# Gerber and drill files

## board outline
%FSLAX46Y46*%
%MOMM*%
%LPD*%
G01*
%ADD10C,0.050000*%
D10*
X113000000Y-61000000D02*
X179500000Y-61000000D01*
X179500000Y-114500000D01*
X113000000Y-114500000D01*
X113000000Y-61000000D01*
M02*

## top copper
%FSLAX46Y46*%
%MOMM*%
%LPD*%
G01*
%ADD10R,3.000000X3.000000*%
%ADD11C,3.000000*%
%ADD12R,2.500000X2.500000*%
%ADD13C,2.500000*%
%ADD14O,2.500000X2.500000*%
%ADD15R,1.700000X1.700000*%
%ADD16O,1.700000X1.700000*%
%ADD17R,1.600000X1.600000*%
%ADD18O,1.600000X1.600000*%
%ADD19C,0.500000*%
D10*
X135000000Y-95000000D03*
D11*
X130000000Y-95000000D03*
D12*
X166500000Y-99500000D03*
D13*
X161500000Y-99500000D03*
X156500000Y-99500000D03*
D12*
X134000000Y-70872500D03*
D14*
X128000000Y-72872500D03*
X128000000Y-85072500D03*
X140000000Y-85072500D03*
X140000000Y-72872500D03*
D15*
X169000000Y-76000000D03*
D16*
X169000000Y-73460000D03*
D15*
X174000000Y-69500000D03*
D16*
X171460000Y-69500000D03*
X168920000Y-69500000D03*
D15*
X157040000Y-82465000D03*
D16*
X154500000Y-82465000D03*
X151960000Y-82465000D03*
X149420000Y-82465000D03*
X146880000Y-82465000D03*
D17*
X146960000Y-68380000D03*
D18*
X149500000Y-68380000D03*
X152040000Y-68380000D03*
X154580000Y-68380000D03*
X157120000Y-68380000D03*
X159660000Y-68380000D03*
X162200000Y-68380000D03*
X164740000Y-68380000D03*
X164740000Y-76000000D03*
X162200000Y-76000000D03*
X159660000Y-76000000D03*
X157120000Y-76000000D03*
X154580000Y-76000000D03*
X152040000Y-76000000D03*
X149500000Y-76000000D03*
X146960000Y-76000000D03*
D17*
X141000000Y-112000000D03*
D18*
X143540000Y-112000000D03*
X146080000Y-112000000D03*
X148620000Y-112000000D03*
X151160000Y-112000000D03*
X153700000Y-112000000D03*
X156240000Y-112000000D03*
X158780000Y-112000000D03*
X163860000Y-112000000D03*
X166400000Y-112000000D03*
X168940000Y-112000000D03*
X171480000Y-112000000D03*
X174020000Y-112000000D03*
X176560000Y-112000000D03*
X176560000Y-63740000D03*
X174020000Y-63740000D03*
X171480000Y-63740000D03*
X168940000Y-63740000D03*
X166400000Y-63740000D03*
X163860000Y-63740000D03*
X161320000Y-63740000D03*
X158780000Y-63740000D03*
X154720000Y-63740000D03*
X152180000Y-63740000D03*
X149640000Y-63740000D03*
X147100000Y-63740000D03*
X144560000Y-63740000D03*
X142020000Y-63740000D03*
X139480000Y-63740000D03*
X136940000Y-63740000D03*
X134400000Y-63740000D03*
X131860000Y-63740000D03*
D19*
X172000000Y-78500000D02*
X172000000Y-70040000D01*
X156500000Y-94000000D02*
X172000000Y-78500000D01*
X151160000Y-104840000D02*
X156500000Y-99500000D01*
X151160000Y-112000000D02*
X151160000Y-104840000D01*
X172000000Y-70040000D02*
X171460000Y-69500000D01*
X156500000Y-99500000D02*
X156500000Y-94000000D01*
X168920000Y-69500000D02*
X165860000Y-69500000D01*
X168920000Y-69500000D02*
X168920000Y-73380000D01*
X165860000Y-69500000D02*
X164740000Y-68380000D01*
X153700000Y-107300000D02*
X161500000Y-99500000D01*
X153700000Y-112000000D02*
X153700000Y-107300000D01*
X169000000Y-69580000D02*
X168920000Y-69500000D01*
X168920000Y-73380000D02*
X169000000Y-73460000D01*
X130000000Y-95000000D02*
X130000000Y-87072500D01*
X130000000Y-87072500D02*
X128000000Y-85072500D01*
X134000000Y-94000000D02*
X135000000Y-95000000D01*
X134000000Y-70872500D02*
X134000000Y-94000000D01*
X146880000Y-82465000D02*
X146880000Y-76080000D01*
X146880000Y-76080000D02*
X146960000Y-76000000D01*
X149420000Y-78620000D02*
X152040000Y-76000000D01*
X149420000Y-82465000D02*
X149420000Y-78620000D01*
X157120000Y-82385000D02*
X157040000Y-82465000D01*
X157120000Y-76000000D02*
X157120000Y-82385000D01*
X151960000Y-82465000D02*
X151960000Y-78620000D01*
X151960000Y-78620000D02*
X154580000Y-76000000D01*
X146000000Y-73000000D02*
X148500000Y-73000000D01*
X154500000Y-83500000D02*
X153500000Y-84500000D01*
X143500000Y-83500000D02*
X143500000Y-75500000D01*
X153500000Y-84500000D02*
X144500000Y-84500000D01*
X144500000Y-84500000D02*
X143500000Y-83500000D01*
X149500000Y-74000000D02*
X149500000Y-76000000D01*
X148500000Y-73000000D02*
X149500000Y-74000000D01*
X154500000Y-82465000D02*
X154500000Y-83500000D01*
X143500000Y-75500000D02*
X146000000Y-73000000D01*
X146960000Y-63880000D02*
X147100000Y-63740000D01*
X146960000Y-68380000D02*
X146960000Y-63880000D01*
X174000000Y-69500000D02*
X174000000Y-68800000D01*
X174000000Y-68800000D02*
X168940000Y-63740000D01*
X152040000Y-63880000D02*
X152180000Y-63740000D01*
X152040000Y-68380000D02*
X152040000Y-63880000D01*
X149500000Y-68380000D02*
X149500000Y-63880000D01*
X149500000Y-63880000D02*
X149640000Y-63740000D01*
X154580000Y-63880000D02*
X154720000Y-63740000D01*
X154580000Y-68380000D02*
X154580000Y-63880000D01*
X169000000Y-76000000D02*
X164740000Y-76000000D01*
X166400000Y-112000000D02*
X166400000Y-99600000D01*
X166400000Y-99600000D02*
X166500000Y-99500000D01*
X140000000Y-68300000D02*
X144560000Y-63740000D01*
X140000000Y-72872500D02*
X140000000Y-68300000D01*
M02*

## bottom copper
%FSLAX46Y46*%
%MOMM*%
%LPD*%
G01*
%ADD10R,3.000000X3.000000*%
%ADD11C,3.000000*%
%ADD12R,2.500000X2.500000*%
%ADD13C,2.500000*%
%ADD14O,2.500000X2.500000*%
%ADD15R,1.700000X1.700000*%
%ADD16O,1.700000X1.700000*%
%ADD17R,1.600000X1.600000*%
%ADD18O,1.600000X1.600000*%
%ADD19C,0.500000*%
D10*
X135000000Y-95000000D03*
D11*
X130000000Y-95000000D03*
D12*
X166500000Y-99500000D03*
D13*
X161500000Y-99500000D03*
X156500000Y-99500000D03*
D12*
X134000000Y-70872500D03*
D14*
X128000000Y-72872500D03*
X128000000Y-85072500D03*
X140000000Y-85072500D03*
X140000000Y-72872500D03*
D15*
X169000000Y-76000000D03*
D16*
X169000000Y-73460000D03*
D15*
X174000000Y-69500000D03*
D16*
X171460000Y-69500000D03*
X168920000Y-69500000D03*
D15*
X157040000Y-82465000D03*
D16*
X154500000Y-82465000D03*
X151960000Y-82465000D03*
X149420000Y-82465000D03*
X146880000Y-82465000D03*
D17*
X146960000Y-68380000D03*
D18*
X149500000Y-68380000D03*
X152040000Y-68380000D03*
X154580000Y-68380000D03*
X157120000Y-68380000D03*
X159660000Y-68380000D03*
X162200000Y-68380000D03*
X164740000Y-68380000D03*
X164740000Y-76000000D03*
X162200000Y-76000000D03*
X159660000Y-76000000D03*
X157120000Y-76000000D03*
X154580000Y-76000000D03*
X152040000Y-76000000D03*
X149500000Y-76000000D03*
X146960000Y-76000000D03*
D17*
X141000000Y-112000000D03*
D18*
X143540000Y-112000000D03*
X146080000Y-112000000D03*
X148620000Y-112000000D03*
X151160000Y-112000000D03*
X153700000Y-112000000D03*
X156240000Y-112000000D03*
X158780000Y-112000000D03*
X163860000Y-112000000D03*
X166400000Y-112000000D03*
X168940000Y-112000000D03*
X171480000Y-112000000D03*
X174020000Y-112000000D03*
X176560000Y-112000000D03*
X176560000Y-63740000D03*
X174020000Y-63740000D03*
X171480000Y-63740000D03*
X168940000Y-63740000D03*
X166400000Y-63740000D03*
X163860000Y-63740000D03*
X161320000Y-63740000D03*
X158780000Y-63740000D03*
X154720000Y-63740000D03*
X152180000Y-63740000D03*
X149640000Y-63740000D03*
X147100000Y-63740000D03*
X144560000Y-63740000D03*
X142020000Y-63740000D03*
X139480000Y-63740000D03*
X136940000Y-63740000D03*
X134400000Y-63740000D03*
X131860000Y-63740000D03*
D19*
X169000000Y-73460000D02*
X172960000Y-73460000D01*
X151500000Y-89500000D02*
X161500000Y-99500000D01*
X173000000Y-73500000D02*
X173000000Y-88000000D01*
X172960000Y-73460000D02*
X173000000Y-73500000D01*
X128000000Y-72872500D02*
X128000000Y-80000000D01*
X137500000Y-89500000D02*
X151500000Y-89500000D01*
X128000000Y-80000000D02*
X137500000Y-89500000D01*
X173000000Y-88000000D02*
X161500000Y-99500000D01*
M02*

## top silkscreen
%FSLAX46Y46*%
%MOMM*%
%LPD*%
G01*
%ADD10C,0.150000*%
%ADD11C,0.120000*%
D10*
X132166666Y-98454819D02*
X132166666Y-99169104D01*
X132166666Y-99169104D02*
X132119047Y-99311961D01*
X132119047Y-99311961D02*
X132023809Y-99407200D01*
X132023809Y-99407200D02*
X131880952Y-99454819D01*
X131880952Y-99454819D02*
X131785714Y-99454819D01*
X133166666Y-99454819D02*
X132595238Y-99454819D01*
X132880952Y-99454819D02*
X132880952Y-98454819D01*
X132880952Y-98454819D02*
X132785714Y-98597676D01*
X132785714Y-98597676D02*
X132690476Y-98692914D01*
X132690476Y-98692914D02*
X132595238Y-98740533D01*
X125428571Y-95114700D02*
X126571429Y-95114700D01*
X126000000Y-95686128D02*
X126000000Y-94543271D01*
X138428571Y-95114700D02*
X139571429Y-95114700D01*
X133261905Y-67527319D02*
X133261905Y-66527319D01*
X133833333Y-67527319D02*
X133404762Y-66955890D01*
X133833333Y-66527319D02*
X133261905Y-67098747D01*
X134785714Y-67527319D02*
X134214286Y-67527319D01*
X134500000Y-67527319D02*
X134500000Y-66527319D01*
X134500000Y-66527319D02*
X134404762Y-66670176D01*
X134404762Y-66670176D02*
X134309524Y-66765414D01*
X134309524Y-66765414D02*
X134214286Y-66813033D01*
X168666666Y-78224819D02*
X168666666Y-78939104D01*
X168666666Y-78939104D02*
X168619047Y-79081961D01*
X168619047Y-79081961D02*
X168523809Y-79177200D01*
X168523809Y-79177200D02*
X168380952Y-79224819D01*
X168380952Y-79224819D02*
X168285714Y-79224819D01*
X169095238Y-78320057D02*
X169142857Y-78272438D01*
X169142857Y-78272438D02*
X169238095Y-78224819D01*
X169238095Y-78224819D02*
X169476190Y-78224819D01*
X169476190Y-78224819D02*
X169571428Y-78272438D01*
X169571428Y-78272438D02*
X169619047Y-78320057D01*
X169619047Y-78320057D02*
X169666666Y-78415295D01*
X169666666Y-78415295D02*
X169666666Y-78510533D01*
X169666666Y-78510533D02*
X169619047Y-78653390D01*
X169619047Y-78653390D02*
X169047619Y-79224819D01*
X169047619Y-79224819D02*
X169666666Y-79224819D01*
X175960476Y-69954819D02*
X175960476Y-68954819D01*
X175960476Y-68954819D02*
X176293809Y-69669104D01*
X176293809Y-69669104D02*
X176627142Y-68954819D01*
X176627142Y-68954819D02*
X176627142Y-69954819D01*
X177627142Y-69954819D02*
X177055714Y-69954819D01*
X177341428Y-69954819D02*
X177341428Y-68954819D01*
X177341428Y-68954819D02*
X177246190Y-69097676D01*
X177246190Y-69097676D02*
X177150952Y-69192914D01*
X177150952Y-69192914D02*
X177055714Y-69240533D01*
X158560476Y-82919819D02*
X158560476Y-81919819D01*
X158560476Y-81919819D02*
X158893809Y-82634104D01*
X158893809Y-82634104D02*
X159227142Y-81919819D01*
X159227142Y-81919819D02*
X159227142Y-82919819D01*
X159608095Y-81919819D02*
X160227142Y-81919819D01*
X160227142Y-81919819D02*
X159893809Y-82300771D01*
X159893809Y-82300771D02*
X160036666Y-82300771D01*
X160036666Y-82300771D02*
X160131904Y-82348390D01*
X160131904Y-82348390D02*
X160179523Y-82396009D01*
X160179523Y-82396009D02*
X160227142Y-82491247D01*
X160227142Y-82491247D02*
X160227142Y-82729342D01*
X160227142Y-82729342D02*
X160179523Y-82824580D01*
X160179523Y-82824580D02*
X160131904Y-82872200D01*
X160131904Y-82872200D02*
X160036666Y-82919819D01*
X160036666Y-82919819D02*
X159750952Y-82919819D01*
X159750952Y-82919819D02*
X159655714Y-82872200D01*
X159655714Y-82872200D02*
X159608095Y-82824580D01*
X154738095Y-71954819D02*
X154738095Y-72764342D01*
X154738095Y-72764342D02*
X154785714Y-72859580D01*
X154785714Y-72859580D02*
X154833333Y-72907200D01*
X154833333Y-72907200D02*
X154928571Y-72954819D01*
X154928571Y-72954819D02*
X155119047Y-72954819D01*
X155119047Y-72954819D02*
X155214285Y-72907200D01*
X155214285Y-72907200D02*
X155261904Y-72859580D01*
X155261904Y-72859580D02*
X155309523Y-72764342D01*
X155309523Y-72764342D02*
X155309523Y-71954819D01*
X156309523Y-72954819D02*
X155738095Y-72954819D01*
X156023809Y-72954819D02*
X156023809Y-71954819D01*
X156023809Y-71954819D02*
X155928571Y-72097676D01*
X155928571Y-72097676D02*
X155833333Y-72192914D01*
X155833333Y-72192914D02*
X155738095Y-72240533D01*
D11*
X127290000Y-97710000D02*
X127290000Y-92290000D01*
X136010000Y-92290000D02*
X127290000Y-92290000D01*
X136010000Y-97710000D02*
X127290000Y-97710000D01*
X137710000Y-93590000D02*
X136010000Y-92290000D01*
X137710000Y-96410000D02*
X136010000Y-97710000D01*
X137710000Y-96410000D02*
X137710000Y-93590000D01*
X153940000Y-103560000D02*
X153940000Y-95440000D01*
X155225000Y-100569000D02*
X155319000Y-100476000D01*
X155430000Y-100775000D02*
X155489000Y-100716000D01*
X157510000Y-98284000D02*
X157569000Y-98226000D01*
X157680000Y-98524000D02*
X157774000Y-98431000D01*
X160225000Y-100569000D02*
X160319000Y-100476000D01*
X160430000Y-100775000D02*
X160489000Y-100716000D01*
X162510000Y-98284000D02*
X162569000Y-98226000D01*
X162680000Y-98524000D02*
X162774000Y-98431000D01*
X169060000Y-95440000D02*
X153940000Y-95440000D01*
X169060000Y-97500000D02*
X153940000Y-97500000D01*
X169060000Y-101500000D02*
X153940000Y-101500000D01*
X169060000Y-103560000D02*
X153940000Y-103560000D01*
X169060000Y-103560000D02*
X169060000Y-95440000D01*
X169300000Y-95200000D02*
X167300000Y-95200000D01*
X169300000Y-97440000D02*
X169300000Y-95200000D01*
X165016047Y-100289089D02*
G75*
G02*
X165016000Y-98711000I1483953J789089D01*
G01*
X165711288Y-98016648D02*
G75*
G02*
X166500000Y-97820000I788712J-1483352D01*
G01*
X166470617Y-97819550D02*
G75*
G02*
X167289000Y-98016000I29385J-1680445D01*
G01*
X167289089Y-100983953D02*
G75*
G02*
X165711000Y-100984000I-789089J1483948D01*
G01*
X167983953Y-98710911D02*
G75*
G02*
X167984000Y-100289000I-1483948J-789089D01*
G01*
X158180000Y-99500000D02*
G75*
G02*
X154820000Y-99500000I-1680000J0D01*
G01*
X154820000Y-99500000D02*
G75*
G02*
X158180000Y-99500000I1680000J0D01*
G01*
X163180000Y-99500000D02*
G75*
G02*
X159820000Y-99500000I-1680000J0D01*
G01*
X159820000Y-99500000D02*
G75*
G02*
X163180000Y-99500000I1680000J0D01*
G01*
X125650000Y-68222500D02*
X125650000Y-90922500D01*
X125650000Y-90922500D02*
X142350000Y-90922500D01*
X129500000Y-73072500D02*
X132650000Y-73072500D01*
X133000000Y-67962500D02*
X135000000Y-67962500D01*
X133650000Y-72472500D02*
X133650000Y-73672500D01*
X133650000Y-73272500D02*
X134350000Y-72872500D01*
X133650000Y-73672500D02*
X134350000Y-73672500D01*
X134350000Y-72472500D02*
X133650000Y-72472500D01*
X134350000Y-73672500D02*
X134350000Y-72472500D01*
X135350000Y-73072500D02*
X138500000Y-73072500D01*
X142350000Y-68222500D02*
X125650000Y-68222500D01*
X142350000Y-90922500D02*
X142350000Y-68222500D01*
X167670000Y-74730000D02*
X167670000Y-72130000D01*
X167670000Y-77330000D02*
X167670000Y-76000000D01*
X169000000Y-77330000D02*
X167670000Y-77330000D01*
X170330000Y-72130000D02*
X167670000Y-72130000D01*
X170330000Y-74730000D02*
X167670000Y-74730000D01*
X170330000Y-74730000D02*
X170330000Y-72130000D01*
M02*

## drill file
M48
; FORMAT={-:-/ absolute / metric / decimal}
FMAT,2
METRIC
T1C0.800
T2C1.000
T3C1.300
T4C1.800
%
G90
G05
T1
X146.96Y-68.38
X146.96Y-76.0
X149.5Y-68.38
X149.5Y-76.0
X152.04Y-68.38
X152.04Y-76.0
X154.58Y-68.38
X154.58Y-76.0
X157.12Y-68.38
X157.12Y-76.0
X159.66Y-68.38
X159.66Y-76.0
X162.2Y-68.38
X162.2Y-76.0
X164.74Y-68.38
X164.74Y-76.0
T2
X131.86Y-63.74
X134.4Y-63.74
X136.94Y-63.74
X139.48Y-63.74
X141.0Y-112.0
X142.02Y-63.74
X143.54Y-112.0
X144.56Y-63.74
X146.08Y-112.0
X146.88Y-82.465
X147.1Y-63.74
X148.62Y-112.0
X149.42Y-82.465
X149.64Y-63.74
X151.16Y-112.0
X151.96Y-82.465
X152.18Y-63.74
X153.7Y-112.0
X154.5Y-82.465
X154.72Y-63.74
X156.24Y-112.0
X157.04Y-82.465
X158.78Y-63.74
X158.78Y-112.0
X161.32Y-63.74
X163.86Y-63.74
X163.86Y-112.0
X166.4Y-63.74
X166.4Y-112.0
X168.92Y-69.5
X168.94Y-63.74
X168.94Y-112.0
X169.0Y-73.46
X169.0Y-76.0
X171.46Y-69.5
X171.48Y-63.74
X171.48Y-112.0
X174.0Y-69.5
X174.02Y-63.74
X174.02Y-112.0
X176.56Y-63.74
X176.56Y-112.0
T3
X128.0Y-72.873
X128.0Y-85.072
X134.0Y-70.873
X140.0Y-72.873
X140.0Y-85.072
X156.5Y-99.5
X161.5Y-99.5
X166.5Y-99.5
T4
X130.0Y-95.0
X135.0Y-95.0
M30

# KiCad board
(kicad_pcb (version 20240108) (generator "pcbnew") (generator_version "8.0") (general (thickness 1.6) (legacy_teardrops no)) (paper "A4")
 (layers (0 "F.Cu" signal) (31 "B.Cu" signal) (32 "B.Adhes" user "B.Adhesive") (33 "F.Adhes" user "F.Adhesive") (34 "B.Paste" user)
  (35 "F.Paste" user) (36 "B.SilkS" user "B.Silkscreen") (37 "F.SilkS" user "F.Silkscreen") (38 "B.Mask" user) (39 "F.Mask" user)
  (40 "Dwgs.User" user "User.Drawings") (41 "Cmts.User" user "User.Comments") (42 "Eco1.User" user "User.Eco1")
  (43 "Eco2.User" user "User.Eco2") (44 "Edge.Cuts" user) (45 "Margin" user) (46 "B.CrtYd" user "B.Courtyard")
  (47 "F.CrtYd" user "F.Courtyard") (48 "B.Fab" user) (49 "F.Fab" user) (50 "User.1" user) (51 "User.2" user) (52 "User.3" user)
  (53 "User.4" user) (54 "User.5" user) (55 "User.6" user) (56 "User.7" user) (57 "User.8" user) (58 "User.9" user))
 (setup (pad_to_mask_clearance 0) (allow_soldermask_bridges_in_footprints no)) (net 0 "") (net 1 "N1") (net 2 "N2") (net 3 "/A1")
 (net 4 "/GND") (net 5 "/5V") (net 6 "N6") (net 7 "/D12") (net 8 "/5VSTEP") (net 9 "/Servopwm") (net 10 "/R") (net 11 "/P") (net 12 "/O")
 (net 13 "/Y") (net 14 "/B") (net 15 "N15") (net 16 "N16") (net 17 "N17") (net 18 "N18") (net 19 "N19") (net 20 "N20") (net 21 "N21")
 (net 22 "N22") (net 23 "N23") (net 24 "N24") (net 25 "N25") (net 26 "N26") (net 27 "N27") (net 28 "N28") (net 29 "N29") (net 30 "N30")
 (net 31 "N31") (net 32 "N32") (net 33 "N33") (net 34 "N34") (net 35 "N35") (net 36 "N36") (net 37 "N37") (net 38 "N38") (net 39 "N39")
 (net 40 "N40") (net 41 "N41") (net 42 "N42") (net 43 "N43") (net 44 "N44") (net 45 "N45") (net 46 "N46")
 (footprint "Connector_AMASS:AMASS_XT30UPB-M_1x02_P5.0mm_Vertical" (layer "F.Cu") (at 135 95 180)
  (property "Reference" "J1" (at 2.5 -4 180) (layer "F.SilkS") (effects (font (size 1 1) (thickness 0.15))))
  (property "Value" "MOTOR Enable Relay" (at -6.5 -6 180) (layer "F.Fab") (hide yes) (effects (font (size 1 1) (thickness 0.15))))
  (fp_line (start 7.71 -2.71) (end 7.71 2.71) (stroke (width 0.12) (type solid)) (layer "F.SilkS"))
  (fp_line (start -1.01 2.71) (end 7.71 2.71) (stroke (width 0.12) (type solid)) (layer "F.SilkS"))
  (fp_line (start -1.01 -2.71) (end 7.71 -2.71) (stroke (width 0.12) (type solid)) (layer "F.SilkS"))
  (fp_line (start -2.71 1.41) (end -1.01 2.71) (stroke (width 0.12) (type solid)) (layer "F.SilkS"))
  (fp_line (start -2.71 -1.41) (end -1.01 -2.71) (stroke (width 0.12) (type solid)) (layer "F.SilkS"))
  (fp_line (start -2.71 -1.41) (end -2.71 1.41) (stroke (width 0.12) (type solid)) (layer "F.SilkS"))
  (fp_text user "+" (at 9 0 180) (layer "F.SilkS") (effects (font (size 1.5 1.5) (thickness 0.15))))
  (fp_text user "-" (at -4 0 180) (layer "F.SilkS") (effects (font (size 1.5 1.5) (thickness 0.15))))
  (pad "1" thru_hole rect (at 0 0 180) (size 3 3) (drill 1.8) (layers "*.Cu" "*.Mask") (remove_unused_layers no) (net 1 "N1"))
  (pad "2" thru_hole circle (at 5 0 180) (size 3 3) (drill 1.8) (layers "*.Cu" "*.Mask") (remove_unused_layers no) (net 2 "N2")))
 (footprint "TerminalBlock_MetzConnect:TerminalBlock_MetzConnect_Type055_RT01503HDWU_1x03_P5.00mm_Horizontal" (layer "F.Cu")
  (at 166.5 99.5 180)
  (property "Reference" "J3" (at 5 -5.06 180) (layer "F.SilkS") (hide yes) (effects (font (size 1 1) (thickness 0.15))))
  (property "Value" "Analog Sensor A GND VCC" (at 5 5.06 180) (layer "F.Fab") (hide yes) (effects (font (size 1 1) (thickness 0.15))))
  (fp_line (start 12.56 -4.06) (end 12.56 4.06) (stroke (width 0.12) (type solid)) (layer "F.SilkS"))
  (fp_line (start 11.275 -1.069) (end 11.181 -0.976) (stroke (width 0.12) (type solid)) (layer "F.SilkS"))
  (fp_line (start 11.07 -1.275) (end 11.011 -1.216) (stroke (width 0.12) (type solid)) (layer "F.SilkS"))
  (fp_line (start 8.99 1.216) (end 8.931 1.274) (stroke (width 0.12) (type solid)) (layer "F.SilkS"))
  (fp_line (start 8.82 0.976) (end 8.726 1.069) (stroke (width 0.12) (type solid)) (layer "F.SilkS"))
  (fp_line (start 6.275 -1.069) (end 6.181 -0.976) (stroke (width 0.12) (type solid)) (layer "F.SilkS"))
  (fp_line (start 6.07 -1.275) (end 6.011 -1.216) (stroke (width 0.12) (type solid)) (layer "F.SilkS"))
  (fp_line (start 3.99 1.216) (end 3.931 1.274) (stroke (width 0.12) (type solid)) (layer "F.SilkS"))
  (fp_line (start 3.82 0.976) (end 3.726 1.069) (stroke (width 0.12) (type solid)) (layer "F.SilkS"))
  (fp_line (start -2.56 4.06) (end 12.56 4.06) (stroke (width 0.12) (type solid)) (layer "F.SilkS"))
  (fp_line (start -2.56 2) (end 12.56 2) (stroke (width 0.12) (type solid)) (layer "F.SilkS"))
  (fp_line (start -2.56 -2) (end 12.56 -2) (stroke (width 0.12) (type solid)) (layer "F.SilkS"))
  (fp_line (start -2.56 -4.06) (end 12.56 -4.06) (stroke (width 0.12) (type solid)) (layer "F.SilkS"))
  (fp_line (start -2.56 -4.06) (end -2.56 4.06) (stroke (width 0.12) (type solid)) (layer "F.SilkS"))
  (fp_line (start -2.8 4.3) (end -0.8 4.3) (stroke (width 0.12) (type solid)) (layer "F.SilkS"))
  (fp_line (start -2.8 2.06) (end -2.8 4.3) (stroke (width 0.12) (type solid)) (layer "F.SilkS"))
  (fp_arc (start 1.483953 -0.789089) (mid 1.680708 -0.00005) (end 1.484 0.789) (stroke (width 0.12) (type solid)) (layer "F.SilkS"))
  (fp_arc (start 0.788712 1.483352) (mid 0.406429 1.630097) (end 0 1.68) (stroke (width 0.12) (type solid)) (layer "F.SilkS"))
  (fp_arc (start 0.029383 1.68045) (mid -0.392304 1.634281) (end -0.789 1.484) (stroke (width 0.12) (type solid)) (layer "F.SilkS"))
  (fp_arc (start -0.789089 -1.483953) (mid -0.00005 -1.680708) (end 0.789 -1.484) (stroke (width 0.12) (type solid)) (layer "F.SilkS"))
  (fp_arc (start -1.483953 0.789089) (mid -1.680708 0.00005) (end -1.484 -0.789) (stroke (width 0.12) (type solid)) (layer "F.SilkS"))
  (fp_circle (center 10 0) (end 11.68 0) (stroke (width 0.12) (type solid)) (fill none) (layer "F.SilkS"))
  (fp_circle (center 5 0) (end 6.68 0) (stroke (width 0.12) (type solid)) (fill none) (layer "F.SilkS"))
  (pad "1" thru_hole rect (at 0 0 180) (size 2.5 2.5) (drill 1.3) (layers "*.Cu" "*.Mask") (remove_unused_layers no) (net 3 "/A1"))
  (pad "2" thru_hole circle (at 5 0 180) (size 2.5 2.5) (drill 1.3) (layers "*.Cu" "*.Mask") (remove_unused_layers no) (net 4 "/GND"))
  (pad "3" thru_hole circle (at 10 0 180) (size 2.5 2.5) (drill 1.3) (layers "*.Cu" "*.Mask") (remove_unused_layers no) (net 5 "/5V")))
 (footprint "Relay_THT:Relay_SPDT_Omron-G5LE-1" (layer "F.Cu") (at 134 70.8725)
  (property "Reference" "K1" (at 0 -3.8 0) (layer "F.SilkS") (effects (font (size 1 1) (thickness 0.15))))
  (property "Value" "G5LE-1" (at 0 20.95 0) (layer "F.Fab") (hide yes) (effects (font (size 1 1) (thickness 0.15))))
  (fp_line (start -8.35 -2.65) (end -8.35 20.05) (stroke (width 0.12) (type solid)) (layer "F.SilkS"))
  (fp_line (start -8.35 20.05) (end 8.35 20.05) (stroke (width 0.12) (type solid)) (layer "F.SilkS"))
  (fp_line (start -4.5 2.2) (end -1.35 2.2) (stroke (width 0.12) (type solid)) (layer "F.SilkS"))
  (fp_line (start -1 -2.91) (end 1 -2.91) (stroke (width 0.12) (type solid)) (layer "F.SilkS"))
  (fp_line (start -0.35 1.6) (end -0.35 2.8) (stroke (width 0.12) (type solid)) (layer "F.SilkS"))
  (fp_line (start -0.35 2.4) (end 0.35 2) (stroke (width 0.12) (type solid)) (layer "F.SilkS"))
  (fp_line (start -0.35 2.8) (end 0.35 2.8) (stroke (width 0.12) (type solid)) (layer "F.SilkS"))
  (fp_line (start 0.35 1.6) (end -0.35 1.6) (stroke (width 0.12) (type solid)) (layer "F.SilkS"))
  (fp_line (start 0.35 2.8) (end 0.35 1.6) (stroke (width 0.12) (type solid)) (layer "F.SilkS"))
  (fp_line (start 1.35 2.2) (end 4.5 2.2) (stroke (width 0.12) (type solid)) (layer "F.SilkS"))
  (fp_line (start 8.35 -2.65) (end -8.35 -2.65) (stroke (width 0.12) (type solid)) (layer "F.SilkS"))
  (fp_line (start 8.35 20.05) (end 8.35 -2.65) (stroke (width 0.12) (type solid)) (layer "F.SilkS"))
  (pad "1" thru_hole rect (at 0 0) (size 2.5 2.5) (drill 1.3) (layers "*.Cu" "*.Mask") (remove_unused_layers no) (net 1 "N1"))
  (pad "2" thru_hole oval (at -6 2) (size 2.5 2.5) (drill 1.3) (layers "*.Cu" "*.Mask") (remove_unused_layers no) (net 4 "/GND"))
  (pad "3" thru_hole oval (at -6 14.2) (size 2.5 2.5) (drill 1.3) (layers "*.Cu" "*.Mask") (remove_unused_layers no) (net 2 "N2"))
  (pad "4" thru_hole oval (at 6 14.2) (size 2.5 2.5) (drill 1.3) (layers "*.Cu" "*.Mask") (remove_unused_layers no) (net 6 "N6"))
  (pad "5" thru_hole oval (at 6 2) (size 2.5 2.5) (drill 1.3) (layers "*.Cu" "*.Mask") (remove_unused_layers no) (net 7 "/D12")))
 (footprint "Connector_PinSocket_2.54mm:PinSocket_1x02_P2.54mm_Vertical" (layer "F.Cu") (at 169 76 180)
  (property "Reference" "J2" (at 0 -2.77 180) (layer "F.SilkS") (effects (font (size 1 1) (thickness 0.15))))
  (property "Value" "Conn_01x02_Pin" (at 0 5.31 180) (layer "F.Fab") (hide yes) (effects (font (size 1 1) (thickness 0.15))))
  (fp_line (start 1.33 1.27) (end 1.33 3.87) (stroke (width 0.12) (type solid)) (layer "F.SilkS"))
  (fp_line (start 1.33 -1.33) (end 1.33 0) (stroke (width 0.12) (type solid)) (layer "F.SilkS"))
  (fp_line (start 0 -1.33) (end 1.33 -1.33) (stroke (width 0.12) (type solid)) (layer "F.SilkS"))
  (fp_line (start -1.33 3.87) (end 1.33 3.87) (stroke (width 0.12) (type solid)) (layer "F.SilkS"))
  (fp_line (start -1.33 1.27) (end 1.33 1.27) (stroke (width 0.12) (type solid)) (layer "F.SilkS"))
  (fp_line (start -1.33 1.27) (end -1.33 3.87) (stroke (width 0.12) (type solid)) (layer "F.SilkS"))
  (pad "1" thru_hole rect (at 0 0 180) (size 1.7 1.7) (drill 1) (layers "*.Cu" "*.Mask") (remove_unused_layers no) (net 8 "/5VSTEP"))
  (pad "2" thru_hole oval (at 0 2.54 180) (size 1.7 1.7) (drill 1) (layers "*.Cu" "*.Mask") (remove_unused_layers no) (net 4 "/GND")))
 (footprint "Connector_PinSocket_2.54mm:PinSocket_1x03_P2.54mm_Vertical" (layer "B.Cu") (at 174 69.5 90)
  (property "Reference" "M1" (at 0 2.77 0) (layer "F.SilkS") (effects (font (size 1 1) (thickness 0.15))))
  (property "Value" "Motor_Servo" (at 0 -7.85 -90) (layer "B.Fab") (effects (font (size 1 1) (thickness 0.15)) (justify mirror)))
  (pad "1" thru_hole rect (at 0 0 90) (size 1.7 1.7) (drill 1) (layers "*.Cu" "*.Mask") (remove_unused_layers no) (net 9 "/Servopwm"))
  (pad "2" thru_hole oval (at 0 -2.54 90) (size 1.7 1.7) (drill 1) (layers "*.Cu" "*.Mask") (remove_unused_layers no) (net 5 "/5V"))
  (pad "3" thru_hole oval (at 0 -5.08 90) (size 1.7 1.7) (drill 1) (layers "*.Cu" "*.Mask") (remove_unused_layers no) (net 4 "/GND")))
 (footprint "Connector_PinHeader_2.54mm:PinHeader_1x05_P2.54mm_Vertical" (layer "B.Cu") (at 157.04 82.465 90)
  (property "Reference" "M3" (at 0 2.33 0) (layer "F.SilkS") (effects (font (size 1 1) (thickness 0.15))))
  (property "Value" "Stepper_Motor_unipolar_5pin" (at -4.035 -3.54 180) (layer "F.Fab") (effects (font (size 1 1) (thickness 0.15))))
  (pad "1" thru_hole rect (at 0 0 90) (size 1.7 1.7) (drill 1) (layers "*.Cu" "*.Mask") (remove_unused_layers no) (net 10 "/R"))
  (pad "2" thru_hole oval (at 0 -2.54 90) (size 1.7 1.7) (drill 1) (layers "*.Cu" "*.Mask") (remove_unused_layers no) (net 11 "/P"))
  (pad "3" thru_hole oval (at 0 -5.08 90) (size 1.7 1.7) (drill 1) (layers "*.Cu" "*.Mask") (remove_unused_layers no) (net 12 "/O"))
  (pad "4" thru_hole oval (at 0 -7.62 90) (size 1.7 1.7) (drill 1) (layers "*.Cu" "*.Mask") (remove_unused_layers no) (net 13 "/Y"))
  (pad "5" thru_hole oval (at 0 -10.16 90) (size 1.7 1.7) (drill 1) (layers "*.Cu" "*.Mask") (remove_unused_layers no) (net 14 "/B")))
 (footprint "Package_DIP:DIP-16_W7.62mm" (layer "B.Cu") (at 146.96 68.38 -90)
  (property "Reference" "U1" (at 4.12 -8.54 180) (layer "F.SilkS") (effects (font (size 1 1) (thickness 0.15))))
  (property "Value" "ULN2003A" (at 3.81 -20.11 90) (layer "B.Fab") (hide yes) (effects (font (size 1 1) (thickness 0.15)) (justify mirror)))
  (pad "1" thru_hole rect (at 0 0 270) (size 1.6 1.6) (drill 0.8) (layers "*.Cu" "*.Mask") (remove_unused_layers no) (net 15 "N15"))
  (pad "2" thru_hole oval (at 0 -2.54 270) (size 1.6 1.6) (drill 0.8) (layers "*.Cu" "*.Mask") (remove_unused_layers no) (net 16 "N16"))
  (pad "3" thru_hole oval (at 0 -5.08 270) (size 1.6 1.6) (drill 0.8) (layers "*.Cu" "*.Mask") (remove_unused_layers no) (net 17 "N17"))
  (pad "4" thru_hole oval (at 0 -7.62 270) (size 1.6 1.6) (drill 0.8) (layers "*.Cu" "*.Mask") (remove_unused_layers no) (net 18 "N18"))
  (pad "5" thru_hole oval (at 0 -10.16 270) (size 1.6 1.6) (drill 0.8) (layers "*.Cu" "*.Mask") (remove_unused_layers no) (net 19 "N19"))
  (pad "6" thru_hole oval (at 0 -12.7 270) (size 1.6 1.6) (drill 0.8) (layers "*.Cu" "*.Mask") (remove_unused_layers no) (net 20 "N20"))
  (pad "7" thru_hole oval (at 0 -15.24 270) (size 1.6 1.6) (drill 0.8) (layers "*.Cu" "*.Mask") (remove_unused_layers no) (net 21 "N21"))
  (pad "8" thru_hole oval (at 0 -17.78 270) (size 1.6 1.6) (drill 0.8) (layers "*.Cu" "*.Mask") (remove_unused_layers no) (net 4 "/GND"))
  (pad "9" thru_hole oval (at 7.62 -17.78 270) (size 1.6 1.6) (drill 0.8) (layers "*.Cu" "*.Mask") (remove_unused_layers no)
   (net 8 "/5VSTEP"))
  (pad "10" thru_hole oval (at 7.62 -15.24 270) (size 1.6 1.6) (drill 0.8) (layers "*.Cu" "*.Mask") (remove_unused_layers no) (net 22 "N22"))
  (pad "11" thru_hole oval (at 7.62 -12.7 270) (size 1.6 1.6) (drill 0.8) (layers "*.Cu" "*.Mask") (remove_unused_layers no) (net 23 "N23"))
  (pad "12" thru_hole oval (at 7.62 -10.16 270) (size 1.6 1.6) (drill 0.8) (layers "*.Cu" "*.Mask") (remove_unused_layers no) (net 10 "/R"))
  (pad "13" thru_hole oval (at 7.62 -7.62 270) (size 1.6 1.6) (drill 0.8) (layers "*.Cu" "*.Mask") (remove_unused_layers no) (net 12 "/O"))
  (pad "14" thru_hole oval (at 7.62 -5.08 270) (size 1.6 1.6) (drill 0.8) (layers "*.Cu" "*.Mask") (remove_unused_layers no) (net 13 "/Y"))
  (pad "15" thru_hole oval (at 7.62 -2.54 270) (size 1.6 1.6) (drill 0.8) (layers "*.Cu" "*.Mask") (remove_unused_layers no) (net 11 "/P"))
  (pad "16" thru_hole oval (at 7.62 0 270) (size 1.6 1.6) (drill 0.8) (layers "*.Cu" "*.Mask") (remove_unused_layers no) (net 14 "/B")))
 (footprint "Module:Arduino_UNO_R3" (layer "B.Cu") (at 141 112)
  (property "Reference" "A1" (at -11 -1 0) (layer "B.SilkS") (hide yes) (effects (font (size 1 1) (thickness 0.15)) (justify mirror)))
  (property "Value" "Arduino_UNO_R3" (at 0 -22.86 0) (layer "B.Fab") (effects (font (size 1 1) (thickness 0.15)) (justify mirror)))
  (pad "1" thru_hole rect (at 0 0 270) (size 1.6 1.6) (drill 1) (layers "*.Cu" "*.Mask") (remove_unused_layers no) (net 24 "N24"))
  (pad "2" thru_hole oval (at 2.54 0 270) (size 1.6 1.6) (drill 1) (layers "*.Cu" "*.Mask") (remove_unused_layers no) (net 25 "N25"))
  (pad "3" thru_hole oval (at 5.08 0 270) (size 1.6 1.6) (drill 1) (layers "*.Cu" "*.Mask") (remove_unused_layers no) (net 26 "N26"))
  (pad "4" thru_hole oval (at 7.62 0 270) (size 1.6 1.6) (drill 1) (layers "*.Cu" "*.Mask") (remove_unused_layers no) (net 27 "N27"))
  (pad "5" thru_hole oval (at 10.16 0 270) (size 1.6 1.6) (drill 1) (layers "*.Cu" "*.Mask") (remove_unused_layers no) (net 5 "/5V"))
  (pad "6" thru_hole oval (at 12.7 0 270) (size 1.6 1.6) (drill 1) (layers "*.Cu" "*.Mask") (remove_unused_layers no) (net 4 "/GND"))
  (pad "7" thru_hole oval (at 15.24 0 270) (size 1.6 1.6) (drill 1) (layers "*.Cu" "*.Mask") (remove_unused_layers no) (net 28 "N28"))
  (pad "8" thru_hole oval (at 17.78 0 270) (size 1.6 1.6) (drill 1) (layers "*.Cu" "*.Mask") (remove_unused_layers no) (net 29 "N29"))
  (pad "9" thru_hole oval (at 22.86 0 270) (size 1.6 1.6) (drill 1) (layers "*.Cu" "*.Mask") (remove_unused_layers no) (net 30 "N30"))
  (pad "10" thru_hole oval (at 25.4 0 270) (size 1.6 1.6) (drill 1) (layers "*.Cu" "*.Mask") (remove_unused_layers no) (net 3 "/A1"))
  (pad "11" thru_hole oval (at 27.94 0 270) (size 1.6 1.6) (drill 1) (layers "*.Cu" "*.Mask") (remove_unused_layers no) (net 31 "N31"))
  (pad "12" thru_hole oval (at 30.48 0 270) (size 1.6 1.6) (drill 1) (layers "*.Cu" "*.Mask") (remove_unused_layers no) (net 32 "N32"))
  (pad "13" thru_hole oval (at 33.02 0 270) (size 1.6 1.6) (drill 1) (layers "*.Cu" "*.Mask") (remove_unused_layers no) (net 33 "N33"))
  (pad "14" thru_hole oval (at 35.56 0 270) (size 1.6 1.6) (drill 1) (layers "*.Cu" "*.Mask") (remove_unused_layers no) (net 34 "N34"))
  (pad "15" thru_hole oval (at 35.56 -48.26 270) (size 1.6 1.6) (drill 1) (layers "*.Cu" "*.Mask") (remove_unused_layers no) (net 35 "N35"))
  (pad "16" thru_hole oval (at 33.02 -48.26 270) (size 1.6 1.6) (drill 1) (layers "*.Cu" "*.Mask") (remove_unused_layers no) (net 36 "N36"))
  (pad "17" thru_hole oval (at 30.48 -48.26 270) (size 1.6 1.6) (drill 1) (layers "*.Cu" "*.Mask") (remove_unused_layers no) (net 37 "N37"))
  (pad "18" thru_hole oval (at 27.94 -48.26 270) (size 1.6 1.6) (drill 1) (layers "*.Cu" "*.Mask") (remove_unused_layers no)
   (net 9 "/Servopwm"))
  (pad "19" thru_hole oval (at 25.4 -48.26 270) (size 1.6 1.6) (drill 1) (layers "*.Cu" "*.Mask") (remove_unused_layers no) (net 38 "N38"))
  (pad "20" thru_hole oval (at 22.86 -48.26 270) (size 1.6 1.6) (drill 1) (layers "*.Cu" "*.Mask") (remove_unused_layers no) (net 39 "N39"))
  (pad "21" thru_hole oval (at 20.32 -48.26 270) (size 1.6 1.6) (drill 1) (layers "*.Cu" "*.Mask") (remove_unused_layers no) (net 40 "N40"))
  (pad "22" thru_hole oval (at 17.78 -48.26 270) (size 1.6 1.6) (drill 1) (layers "*.Cu" "*.Mask") (remove_unused_layers no) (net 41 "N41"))
  (pad "23" thru_hole oval (at 13.72 -48.26 270) (size 1.6 1.6) (drill 1) (layers "*.Cu" "*.Mask") (remove_unused_layers no) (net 18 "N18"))
  (pad "24" thru_hole oval (at 11.18 -48.26 270) (size 1.6 1.6) (drill 1) (layers "*.Cu" "*.Mask") (remove_unused_layers no) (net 17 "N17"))
  (pad "25" thru_hole oval (at 8.64 -48.26 270) (size 1.6 1.6) (drill 1) (layers "*.Cu" "*.Mask") (remove_unused_layers no) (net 16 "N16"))
  (pad "26" thru_hole oval (at 6.1 -48.26 270) (size 1.6 1.6) (drill 1) (layers "*.Cu" "*.Mask") (remove_unused_layers no) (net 15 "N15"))
  (pad "27" thru_hole oval (at 3.56 -48.26 270) (size 1.6 1.6) (drill 1) (layers "*.Cu" "*.Mask") (remove_unused_layers no) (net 7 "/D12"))
  (pad "28" thru_hole oval (at 1.02 -48.26 270) (size 1.6 1.6) (drill 1) (layers "*.Cu" "*.Mask") (remove_unused_layers no) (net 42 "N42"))
  (pad "29" thru_hole oval (at -1.52 -48.26 270) (size 1.6 1.6) (drill 1) (layers "*.Cu" "*.Mask") (remove_unused_layers no) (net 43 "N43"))
  (pad "30" thru_hole oval (at -4.06 -48.26 270) (size 1.6 1.6) (drill 1) (layers "*.Cu" "*.Mask") (remove_unused_layers no) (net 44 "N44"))
  (pad "31" thru_hole oval (at -6.6 -48.26 270) (size 1.6 1.6) (drill 1) (layers "*.Cu" "*.Mask") (remove_unused_layers no) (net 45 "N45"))
  (pad "32" thru_hole oval (at -9.14 -48.26 270) (size 1.6 1.6) (drill 1) (layers "*.Cu" "*.Mask") (remove_unused_layers no) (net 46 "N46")))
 (gr_rect (start 113 61) (end 179.5 114.5) (stroke (width 0.05) (type default)) (fill none) (layer "Edge.Cuts"))
 (segment (start 172 78.5) (end 172 70.04) (width 0.5) (layer "F.Cu") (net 5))
 (segment (start 156.5 94) (end 172 78.5) (width 0.5) (layer "F.Cu") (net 5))
 (segment (start 151.16 104.84) (end 156.5 99.5) (width 0.5) (layer "F.Cu") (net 5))
 (segment (start 151.16 112) (end 151.16 104.84) (width 0.5) (layer "F.Cu") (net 5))
 (segment (start 172 70.04) (end 171.46 69.5) (width 0.5) (layer "F.Cu") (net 5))
 (segment (start 156.5 99.5) (end 156.5 94) (width 0.5) (layer "F.Cu") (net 5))
 (segment (start 168.92 69.5) (end 165.86 69.5) (width 0.5) (layer "F.Cu") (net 4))
 (segment (start 168.92 69.5) (end 168.92 73.38) (width 0.5) (layer "F.Cu") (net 4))
 (segment (start 165.86 69.5) (end 164.74 68.38) (width 0.5) (layer "F.Cu") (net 4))
 (segment (start 153.7 107.3) (end 161.5 99.5) (width 0.5) (layer "F.Cu") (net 4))
 (segment (start 153.7 112) (end 153.7 107.3) (width 0.5) (layer "F.Cu") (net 4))
 (segment (start 169 69.58) (end 168.92 69.5) (width 0.5) (layer "F.Cu") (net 4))
 (segment (start 168.92 73.38) (end 169 73.46) (width 0.5) (layer "F.Cu") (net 4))
 (segment (start 169 73.46) (end 172.96 73.46) (width 0.5) (layer "B.Cu") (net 4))
 (segment (start 151.5 89.5) (end 161.5 99.5) (width 0.5) (layer "B.Cu") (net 4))
 (segment (start 173 73.5) (end 173 88) (width 0.5) (layer "B.Cu") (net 4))
 (segment (start 172.96 73.46) (end 173 73.5) (width 0.5) (layer "B.Cu") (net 4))
 (segment (start 128 72.8725) (end 128 80) (width 0.5) (layer "B.Cu") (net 4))
 (segment (start 137.5 89.5) (end 151.5 89.5) (width 0.5) (layer "B.Cu") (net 4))
 (segment (start 128 80) (end 137.5 89.5) (width 0.5) (layer "B.Cu") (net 4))
 (segment (start 173 88) (end 161.5 99.5) (width 0.5) (layer "B.Cu") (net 4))
 (segment (start 130 95) (end 130 87.0725) (width 0.5) (layer "F.Cu") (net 2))
 (segment (start 130 87.0725) (end 128 85.0725) (width 0.5) (layer "F.Cu") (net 2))
 (segment (start 134 94) (end 135 95) (width 0.5) (layer "F.Cu") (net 1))
 (segment (start 134 70.8725) (end 134 94) (width 0.5) (layer "F.Cu") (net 1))
 (segment (start 146.88 82.465) (end 146.88 76.08) (width 0.5) (layer "F.Cu") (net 14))
 (segment (start 146.88 76.08) (end 146.96 76) (width 0.5) (layer "F.Cu") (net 14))
 (segment (start 149.42 78.62) (end 152.04 76) (width 0.5) (layer "F.Cu") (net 13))
 (segment (start 149.42 82.465) (end 149.42 78.62) (width 0.5) (layer "F.Cu") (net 13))
 (segment (start 157.12 82.385) (end 157.04 82.465) (width 0.5) (layer "F.Cu") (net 10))
 (segment (start 157.12 76) (end 157.12 82.385) (width 0.5) (layer "F.Cu") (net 10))
 (segment (start 151.96 82.465) (end 151.96 78.62) (width 0.5) (layer "F.Cu") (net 12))
 (segment (start 151.96 78.62) (end 154.58 76) (width 0.5) (layer "F.Cu") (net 12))
 (segment (start 146 73) (end 148.5 73) (width 0.5) (layer "F.Cu") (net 11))
 (segment (start 154.5 83.5) (end 153.5 84.5) (width 0.5) (layer "F.Cu") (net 11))
 (segment (start 143.5 83.5) (end 143.5 75.5) (width 0.5) (layer "F.Cu") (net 11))
 (segment (start 153.5 84.5) (end 144.5 84.5) (width 0.5) (layer "F.Cu") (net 11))
 (segment (start 144.5 84.5) (end 143.5 83.5) (width 0.5) (layer "F.Cu") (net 11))
 (segment (start 149.5 74) (end 149.5 76) (width 0.5) (layer "F.Cu") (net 11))
 (segment (start 148.5 73) (end 149.5 74) (width 0.5) (layer "F.Cu") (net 11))
 (segment (start 154.5 82.465) (end 154.5 83.5) (width 0.5) (layer "F.Cu") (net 11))
 (segment (start 143.5 75.5) (end 146 73) (width 0.5) (layer "F.Cu") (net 11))
 (segment (start 146.96 63.88) (end 147.1 63.74) (width 0.5) (layer "F.Cu") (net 15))
 (segment (start 146.96 68.38) (end 146.96 63.88) (width 0.5) (layer "F.Cu") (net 15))
 (segment (start 174 69.5) (end 174 68.8) (width 0.5) (layer "F.Cu") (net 9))
 (segment (start 174 68.8) (end 168.94 63.74) (width 0.5) (layer "F.Cu") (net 9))
 (segment (start 152.04 63.88) (end 152.18 63.74) (width 0.5) (layer "F.Cu") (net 17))
 (segment (start 152.04 68.38) (end 152.04 63.88) (width 0.5) (layer "F.Cu") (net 17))
 (segment (start 149.5 68.38) (end 149.5 63.88) (width 0.5) (layer "F.Cu") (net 16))
 (segment (start 149.5 63.88) (end 149.64 63.74) (width 0.5) (layer "F.Cu") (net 16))
 (segment (start 154.58 63.88) (end 154.72 63.74) (width 0.5) (layer "F.Cu") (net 18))
 (segment (start 154.58 68.38) (end 154.58 63.88) (width 0.5) (layer "F.Cu") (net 18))
 (segment (start 169 76) (end 164.74 76) (width 0.5) (layer "F.Cu") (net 8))
 (segment (start 166.4 112) (end 166.4 99.6) (width 0.5) (layer "F.Cu") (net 3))
 (segment (start 166.4 99.6) (end 166.5 99.5) (width 0.5) (layer "F.Cu") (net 3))
 (segment (start 140 68.3) (end 144.56 63.74) (width 0.5) (layer "F.Cu") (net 7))
 (segment (start 140 72.8725) (end 140 68.3) (width 0.5) (layer "F.Cu") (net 7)))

